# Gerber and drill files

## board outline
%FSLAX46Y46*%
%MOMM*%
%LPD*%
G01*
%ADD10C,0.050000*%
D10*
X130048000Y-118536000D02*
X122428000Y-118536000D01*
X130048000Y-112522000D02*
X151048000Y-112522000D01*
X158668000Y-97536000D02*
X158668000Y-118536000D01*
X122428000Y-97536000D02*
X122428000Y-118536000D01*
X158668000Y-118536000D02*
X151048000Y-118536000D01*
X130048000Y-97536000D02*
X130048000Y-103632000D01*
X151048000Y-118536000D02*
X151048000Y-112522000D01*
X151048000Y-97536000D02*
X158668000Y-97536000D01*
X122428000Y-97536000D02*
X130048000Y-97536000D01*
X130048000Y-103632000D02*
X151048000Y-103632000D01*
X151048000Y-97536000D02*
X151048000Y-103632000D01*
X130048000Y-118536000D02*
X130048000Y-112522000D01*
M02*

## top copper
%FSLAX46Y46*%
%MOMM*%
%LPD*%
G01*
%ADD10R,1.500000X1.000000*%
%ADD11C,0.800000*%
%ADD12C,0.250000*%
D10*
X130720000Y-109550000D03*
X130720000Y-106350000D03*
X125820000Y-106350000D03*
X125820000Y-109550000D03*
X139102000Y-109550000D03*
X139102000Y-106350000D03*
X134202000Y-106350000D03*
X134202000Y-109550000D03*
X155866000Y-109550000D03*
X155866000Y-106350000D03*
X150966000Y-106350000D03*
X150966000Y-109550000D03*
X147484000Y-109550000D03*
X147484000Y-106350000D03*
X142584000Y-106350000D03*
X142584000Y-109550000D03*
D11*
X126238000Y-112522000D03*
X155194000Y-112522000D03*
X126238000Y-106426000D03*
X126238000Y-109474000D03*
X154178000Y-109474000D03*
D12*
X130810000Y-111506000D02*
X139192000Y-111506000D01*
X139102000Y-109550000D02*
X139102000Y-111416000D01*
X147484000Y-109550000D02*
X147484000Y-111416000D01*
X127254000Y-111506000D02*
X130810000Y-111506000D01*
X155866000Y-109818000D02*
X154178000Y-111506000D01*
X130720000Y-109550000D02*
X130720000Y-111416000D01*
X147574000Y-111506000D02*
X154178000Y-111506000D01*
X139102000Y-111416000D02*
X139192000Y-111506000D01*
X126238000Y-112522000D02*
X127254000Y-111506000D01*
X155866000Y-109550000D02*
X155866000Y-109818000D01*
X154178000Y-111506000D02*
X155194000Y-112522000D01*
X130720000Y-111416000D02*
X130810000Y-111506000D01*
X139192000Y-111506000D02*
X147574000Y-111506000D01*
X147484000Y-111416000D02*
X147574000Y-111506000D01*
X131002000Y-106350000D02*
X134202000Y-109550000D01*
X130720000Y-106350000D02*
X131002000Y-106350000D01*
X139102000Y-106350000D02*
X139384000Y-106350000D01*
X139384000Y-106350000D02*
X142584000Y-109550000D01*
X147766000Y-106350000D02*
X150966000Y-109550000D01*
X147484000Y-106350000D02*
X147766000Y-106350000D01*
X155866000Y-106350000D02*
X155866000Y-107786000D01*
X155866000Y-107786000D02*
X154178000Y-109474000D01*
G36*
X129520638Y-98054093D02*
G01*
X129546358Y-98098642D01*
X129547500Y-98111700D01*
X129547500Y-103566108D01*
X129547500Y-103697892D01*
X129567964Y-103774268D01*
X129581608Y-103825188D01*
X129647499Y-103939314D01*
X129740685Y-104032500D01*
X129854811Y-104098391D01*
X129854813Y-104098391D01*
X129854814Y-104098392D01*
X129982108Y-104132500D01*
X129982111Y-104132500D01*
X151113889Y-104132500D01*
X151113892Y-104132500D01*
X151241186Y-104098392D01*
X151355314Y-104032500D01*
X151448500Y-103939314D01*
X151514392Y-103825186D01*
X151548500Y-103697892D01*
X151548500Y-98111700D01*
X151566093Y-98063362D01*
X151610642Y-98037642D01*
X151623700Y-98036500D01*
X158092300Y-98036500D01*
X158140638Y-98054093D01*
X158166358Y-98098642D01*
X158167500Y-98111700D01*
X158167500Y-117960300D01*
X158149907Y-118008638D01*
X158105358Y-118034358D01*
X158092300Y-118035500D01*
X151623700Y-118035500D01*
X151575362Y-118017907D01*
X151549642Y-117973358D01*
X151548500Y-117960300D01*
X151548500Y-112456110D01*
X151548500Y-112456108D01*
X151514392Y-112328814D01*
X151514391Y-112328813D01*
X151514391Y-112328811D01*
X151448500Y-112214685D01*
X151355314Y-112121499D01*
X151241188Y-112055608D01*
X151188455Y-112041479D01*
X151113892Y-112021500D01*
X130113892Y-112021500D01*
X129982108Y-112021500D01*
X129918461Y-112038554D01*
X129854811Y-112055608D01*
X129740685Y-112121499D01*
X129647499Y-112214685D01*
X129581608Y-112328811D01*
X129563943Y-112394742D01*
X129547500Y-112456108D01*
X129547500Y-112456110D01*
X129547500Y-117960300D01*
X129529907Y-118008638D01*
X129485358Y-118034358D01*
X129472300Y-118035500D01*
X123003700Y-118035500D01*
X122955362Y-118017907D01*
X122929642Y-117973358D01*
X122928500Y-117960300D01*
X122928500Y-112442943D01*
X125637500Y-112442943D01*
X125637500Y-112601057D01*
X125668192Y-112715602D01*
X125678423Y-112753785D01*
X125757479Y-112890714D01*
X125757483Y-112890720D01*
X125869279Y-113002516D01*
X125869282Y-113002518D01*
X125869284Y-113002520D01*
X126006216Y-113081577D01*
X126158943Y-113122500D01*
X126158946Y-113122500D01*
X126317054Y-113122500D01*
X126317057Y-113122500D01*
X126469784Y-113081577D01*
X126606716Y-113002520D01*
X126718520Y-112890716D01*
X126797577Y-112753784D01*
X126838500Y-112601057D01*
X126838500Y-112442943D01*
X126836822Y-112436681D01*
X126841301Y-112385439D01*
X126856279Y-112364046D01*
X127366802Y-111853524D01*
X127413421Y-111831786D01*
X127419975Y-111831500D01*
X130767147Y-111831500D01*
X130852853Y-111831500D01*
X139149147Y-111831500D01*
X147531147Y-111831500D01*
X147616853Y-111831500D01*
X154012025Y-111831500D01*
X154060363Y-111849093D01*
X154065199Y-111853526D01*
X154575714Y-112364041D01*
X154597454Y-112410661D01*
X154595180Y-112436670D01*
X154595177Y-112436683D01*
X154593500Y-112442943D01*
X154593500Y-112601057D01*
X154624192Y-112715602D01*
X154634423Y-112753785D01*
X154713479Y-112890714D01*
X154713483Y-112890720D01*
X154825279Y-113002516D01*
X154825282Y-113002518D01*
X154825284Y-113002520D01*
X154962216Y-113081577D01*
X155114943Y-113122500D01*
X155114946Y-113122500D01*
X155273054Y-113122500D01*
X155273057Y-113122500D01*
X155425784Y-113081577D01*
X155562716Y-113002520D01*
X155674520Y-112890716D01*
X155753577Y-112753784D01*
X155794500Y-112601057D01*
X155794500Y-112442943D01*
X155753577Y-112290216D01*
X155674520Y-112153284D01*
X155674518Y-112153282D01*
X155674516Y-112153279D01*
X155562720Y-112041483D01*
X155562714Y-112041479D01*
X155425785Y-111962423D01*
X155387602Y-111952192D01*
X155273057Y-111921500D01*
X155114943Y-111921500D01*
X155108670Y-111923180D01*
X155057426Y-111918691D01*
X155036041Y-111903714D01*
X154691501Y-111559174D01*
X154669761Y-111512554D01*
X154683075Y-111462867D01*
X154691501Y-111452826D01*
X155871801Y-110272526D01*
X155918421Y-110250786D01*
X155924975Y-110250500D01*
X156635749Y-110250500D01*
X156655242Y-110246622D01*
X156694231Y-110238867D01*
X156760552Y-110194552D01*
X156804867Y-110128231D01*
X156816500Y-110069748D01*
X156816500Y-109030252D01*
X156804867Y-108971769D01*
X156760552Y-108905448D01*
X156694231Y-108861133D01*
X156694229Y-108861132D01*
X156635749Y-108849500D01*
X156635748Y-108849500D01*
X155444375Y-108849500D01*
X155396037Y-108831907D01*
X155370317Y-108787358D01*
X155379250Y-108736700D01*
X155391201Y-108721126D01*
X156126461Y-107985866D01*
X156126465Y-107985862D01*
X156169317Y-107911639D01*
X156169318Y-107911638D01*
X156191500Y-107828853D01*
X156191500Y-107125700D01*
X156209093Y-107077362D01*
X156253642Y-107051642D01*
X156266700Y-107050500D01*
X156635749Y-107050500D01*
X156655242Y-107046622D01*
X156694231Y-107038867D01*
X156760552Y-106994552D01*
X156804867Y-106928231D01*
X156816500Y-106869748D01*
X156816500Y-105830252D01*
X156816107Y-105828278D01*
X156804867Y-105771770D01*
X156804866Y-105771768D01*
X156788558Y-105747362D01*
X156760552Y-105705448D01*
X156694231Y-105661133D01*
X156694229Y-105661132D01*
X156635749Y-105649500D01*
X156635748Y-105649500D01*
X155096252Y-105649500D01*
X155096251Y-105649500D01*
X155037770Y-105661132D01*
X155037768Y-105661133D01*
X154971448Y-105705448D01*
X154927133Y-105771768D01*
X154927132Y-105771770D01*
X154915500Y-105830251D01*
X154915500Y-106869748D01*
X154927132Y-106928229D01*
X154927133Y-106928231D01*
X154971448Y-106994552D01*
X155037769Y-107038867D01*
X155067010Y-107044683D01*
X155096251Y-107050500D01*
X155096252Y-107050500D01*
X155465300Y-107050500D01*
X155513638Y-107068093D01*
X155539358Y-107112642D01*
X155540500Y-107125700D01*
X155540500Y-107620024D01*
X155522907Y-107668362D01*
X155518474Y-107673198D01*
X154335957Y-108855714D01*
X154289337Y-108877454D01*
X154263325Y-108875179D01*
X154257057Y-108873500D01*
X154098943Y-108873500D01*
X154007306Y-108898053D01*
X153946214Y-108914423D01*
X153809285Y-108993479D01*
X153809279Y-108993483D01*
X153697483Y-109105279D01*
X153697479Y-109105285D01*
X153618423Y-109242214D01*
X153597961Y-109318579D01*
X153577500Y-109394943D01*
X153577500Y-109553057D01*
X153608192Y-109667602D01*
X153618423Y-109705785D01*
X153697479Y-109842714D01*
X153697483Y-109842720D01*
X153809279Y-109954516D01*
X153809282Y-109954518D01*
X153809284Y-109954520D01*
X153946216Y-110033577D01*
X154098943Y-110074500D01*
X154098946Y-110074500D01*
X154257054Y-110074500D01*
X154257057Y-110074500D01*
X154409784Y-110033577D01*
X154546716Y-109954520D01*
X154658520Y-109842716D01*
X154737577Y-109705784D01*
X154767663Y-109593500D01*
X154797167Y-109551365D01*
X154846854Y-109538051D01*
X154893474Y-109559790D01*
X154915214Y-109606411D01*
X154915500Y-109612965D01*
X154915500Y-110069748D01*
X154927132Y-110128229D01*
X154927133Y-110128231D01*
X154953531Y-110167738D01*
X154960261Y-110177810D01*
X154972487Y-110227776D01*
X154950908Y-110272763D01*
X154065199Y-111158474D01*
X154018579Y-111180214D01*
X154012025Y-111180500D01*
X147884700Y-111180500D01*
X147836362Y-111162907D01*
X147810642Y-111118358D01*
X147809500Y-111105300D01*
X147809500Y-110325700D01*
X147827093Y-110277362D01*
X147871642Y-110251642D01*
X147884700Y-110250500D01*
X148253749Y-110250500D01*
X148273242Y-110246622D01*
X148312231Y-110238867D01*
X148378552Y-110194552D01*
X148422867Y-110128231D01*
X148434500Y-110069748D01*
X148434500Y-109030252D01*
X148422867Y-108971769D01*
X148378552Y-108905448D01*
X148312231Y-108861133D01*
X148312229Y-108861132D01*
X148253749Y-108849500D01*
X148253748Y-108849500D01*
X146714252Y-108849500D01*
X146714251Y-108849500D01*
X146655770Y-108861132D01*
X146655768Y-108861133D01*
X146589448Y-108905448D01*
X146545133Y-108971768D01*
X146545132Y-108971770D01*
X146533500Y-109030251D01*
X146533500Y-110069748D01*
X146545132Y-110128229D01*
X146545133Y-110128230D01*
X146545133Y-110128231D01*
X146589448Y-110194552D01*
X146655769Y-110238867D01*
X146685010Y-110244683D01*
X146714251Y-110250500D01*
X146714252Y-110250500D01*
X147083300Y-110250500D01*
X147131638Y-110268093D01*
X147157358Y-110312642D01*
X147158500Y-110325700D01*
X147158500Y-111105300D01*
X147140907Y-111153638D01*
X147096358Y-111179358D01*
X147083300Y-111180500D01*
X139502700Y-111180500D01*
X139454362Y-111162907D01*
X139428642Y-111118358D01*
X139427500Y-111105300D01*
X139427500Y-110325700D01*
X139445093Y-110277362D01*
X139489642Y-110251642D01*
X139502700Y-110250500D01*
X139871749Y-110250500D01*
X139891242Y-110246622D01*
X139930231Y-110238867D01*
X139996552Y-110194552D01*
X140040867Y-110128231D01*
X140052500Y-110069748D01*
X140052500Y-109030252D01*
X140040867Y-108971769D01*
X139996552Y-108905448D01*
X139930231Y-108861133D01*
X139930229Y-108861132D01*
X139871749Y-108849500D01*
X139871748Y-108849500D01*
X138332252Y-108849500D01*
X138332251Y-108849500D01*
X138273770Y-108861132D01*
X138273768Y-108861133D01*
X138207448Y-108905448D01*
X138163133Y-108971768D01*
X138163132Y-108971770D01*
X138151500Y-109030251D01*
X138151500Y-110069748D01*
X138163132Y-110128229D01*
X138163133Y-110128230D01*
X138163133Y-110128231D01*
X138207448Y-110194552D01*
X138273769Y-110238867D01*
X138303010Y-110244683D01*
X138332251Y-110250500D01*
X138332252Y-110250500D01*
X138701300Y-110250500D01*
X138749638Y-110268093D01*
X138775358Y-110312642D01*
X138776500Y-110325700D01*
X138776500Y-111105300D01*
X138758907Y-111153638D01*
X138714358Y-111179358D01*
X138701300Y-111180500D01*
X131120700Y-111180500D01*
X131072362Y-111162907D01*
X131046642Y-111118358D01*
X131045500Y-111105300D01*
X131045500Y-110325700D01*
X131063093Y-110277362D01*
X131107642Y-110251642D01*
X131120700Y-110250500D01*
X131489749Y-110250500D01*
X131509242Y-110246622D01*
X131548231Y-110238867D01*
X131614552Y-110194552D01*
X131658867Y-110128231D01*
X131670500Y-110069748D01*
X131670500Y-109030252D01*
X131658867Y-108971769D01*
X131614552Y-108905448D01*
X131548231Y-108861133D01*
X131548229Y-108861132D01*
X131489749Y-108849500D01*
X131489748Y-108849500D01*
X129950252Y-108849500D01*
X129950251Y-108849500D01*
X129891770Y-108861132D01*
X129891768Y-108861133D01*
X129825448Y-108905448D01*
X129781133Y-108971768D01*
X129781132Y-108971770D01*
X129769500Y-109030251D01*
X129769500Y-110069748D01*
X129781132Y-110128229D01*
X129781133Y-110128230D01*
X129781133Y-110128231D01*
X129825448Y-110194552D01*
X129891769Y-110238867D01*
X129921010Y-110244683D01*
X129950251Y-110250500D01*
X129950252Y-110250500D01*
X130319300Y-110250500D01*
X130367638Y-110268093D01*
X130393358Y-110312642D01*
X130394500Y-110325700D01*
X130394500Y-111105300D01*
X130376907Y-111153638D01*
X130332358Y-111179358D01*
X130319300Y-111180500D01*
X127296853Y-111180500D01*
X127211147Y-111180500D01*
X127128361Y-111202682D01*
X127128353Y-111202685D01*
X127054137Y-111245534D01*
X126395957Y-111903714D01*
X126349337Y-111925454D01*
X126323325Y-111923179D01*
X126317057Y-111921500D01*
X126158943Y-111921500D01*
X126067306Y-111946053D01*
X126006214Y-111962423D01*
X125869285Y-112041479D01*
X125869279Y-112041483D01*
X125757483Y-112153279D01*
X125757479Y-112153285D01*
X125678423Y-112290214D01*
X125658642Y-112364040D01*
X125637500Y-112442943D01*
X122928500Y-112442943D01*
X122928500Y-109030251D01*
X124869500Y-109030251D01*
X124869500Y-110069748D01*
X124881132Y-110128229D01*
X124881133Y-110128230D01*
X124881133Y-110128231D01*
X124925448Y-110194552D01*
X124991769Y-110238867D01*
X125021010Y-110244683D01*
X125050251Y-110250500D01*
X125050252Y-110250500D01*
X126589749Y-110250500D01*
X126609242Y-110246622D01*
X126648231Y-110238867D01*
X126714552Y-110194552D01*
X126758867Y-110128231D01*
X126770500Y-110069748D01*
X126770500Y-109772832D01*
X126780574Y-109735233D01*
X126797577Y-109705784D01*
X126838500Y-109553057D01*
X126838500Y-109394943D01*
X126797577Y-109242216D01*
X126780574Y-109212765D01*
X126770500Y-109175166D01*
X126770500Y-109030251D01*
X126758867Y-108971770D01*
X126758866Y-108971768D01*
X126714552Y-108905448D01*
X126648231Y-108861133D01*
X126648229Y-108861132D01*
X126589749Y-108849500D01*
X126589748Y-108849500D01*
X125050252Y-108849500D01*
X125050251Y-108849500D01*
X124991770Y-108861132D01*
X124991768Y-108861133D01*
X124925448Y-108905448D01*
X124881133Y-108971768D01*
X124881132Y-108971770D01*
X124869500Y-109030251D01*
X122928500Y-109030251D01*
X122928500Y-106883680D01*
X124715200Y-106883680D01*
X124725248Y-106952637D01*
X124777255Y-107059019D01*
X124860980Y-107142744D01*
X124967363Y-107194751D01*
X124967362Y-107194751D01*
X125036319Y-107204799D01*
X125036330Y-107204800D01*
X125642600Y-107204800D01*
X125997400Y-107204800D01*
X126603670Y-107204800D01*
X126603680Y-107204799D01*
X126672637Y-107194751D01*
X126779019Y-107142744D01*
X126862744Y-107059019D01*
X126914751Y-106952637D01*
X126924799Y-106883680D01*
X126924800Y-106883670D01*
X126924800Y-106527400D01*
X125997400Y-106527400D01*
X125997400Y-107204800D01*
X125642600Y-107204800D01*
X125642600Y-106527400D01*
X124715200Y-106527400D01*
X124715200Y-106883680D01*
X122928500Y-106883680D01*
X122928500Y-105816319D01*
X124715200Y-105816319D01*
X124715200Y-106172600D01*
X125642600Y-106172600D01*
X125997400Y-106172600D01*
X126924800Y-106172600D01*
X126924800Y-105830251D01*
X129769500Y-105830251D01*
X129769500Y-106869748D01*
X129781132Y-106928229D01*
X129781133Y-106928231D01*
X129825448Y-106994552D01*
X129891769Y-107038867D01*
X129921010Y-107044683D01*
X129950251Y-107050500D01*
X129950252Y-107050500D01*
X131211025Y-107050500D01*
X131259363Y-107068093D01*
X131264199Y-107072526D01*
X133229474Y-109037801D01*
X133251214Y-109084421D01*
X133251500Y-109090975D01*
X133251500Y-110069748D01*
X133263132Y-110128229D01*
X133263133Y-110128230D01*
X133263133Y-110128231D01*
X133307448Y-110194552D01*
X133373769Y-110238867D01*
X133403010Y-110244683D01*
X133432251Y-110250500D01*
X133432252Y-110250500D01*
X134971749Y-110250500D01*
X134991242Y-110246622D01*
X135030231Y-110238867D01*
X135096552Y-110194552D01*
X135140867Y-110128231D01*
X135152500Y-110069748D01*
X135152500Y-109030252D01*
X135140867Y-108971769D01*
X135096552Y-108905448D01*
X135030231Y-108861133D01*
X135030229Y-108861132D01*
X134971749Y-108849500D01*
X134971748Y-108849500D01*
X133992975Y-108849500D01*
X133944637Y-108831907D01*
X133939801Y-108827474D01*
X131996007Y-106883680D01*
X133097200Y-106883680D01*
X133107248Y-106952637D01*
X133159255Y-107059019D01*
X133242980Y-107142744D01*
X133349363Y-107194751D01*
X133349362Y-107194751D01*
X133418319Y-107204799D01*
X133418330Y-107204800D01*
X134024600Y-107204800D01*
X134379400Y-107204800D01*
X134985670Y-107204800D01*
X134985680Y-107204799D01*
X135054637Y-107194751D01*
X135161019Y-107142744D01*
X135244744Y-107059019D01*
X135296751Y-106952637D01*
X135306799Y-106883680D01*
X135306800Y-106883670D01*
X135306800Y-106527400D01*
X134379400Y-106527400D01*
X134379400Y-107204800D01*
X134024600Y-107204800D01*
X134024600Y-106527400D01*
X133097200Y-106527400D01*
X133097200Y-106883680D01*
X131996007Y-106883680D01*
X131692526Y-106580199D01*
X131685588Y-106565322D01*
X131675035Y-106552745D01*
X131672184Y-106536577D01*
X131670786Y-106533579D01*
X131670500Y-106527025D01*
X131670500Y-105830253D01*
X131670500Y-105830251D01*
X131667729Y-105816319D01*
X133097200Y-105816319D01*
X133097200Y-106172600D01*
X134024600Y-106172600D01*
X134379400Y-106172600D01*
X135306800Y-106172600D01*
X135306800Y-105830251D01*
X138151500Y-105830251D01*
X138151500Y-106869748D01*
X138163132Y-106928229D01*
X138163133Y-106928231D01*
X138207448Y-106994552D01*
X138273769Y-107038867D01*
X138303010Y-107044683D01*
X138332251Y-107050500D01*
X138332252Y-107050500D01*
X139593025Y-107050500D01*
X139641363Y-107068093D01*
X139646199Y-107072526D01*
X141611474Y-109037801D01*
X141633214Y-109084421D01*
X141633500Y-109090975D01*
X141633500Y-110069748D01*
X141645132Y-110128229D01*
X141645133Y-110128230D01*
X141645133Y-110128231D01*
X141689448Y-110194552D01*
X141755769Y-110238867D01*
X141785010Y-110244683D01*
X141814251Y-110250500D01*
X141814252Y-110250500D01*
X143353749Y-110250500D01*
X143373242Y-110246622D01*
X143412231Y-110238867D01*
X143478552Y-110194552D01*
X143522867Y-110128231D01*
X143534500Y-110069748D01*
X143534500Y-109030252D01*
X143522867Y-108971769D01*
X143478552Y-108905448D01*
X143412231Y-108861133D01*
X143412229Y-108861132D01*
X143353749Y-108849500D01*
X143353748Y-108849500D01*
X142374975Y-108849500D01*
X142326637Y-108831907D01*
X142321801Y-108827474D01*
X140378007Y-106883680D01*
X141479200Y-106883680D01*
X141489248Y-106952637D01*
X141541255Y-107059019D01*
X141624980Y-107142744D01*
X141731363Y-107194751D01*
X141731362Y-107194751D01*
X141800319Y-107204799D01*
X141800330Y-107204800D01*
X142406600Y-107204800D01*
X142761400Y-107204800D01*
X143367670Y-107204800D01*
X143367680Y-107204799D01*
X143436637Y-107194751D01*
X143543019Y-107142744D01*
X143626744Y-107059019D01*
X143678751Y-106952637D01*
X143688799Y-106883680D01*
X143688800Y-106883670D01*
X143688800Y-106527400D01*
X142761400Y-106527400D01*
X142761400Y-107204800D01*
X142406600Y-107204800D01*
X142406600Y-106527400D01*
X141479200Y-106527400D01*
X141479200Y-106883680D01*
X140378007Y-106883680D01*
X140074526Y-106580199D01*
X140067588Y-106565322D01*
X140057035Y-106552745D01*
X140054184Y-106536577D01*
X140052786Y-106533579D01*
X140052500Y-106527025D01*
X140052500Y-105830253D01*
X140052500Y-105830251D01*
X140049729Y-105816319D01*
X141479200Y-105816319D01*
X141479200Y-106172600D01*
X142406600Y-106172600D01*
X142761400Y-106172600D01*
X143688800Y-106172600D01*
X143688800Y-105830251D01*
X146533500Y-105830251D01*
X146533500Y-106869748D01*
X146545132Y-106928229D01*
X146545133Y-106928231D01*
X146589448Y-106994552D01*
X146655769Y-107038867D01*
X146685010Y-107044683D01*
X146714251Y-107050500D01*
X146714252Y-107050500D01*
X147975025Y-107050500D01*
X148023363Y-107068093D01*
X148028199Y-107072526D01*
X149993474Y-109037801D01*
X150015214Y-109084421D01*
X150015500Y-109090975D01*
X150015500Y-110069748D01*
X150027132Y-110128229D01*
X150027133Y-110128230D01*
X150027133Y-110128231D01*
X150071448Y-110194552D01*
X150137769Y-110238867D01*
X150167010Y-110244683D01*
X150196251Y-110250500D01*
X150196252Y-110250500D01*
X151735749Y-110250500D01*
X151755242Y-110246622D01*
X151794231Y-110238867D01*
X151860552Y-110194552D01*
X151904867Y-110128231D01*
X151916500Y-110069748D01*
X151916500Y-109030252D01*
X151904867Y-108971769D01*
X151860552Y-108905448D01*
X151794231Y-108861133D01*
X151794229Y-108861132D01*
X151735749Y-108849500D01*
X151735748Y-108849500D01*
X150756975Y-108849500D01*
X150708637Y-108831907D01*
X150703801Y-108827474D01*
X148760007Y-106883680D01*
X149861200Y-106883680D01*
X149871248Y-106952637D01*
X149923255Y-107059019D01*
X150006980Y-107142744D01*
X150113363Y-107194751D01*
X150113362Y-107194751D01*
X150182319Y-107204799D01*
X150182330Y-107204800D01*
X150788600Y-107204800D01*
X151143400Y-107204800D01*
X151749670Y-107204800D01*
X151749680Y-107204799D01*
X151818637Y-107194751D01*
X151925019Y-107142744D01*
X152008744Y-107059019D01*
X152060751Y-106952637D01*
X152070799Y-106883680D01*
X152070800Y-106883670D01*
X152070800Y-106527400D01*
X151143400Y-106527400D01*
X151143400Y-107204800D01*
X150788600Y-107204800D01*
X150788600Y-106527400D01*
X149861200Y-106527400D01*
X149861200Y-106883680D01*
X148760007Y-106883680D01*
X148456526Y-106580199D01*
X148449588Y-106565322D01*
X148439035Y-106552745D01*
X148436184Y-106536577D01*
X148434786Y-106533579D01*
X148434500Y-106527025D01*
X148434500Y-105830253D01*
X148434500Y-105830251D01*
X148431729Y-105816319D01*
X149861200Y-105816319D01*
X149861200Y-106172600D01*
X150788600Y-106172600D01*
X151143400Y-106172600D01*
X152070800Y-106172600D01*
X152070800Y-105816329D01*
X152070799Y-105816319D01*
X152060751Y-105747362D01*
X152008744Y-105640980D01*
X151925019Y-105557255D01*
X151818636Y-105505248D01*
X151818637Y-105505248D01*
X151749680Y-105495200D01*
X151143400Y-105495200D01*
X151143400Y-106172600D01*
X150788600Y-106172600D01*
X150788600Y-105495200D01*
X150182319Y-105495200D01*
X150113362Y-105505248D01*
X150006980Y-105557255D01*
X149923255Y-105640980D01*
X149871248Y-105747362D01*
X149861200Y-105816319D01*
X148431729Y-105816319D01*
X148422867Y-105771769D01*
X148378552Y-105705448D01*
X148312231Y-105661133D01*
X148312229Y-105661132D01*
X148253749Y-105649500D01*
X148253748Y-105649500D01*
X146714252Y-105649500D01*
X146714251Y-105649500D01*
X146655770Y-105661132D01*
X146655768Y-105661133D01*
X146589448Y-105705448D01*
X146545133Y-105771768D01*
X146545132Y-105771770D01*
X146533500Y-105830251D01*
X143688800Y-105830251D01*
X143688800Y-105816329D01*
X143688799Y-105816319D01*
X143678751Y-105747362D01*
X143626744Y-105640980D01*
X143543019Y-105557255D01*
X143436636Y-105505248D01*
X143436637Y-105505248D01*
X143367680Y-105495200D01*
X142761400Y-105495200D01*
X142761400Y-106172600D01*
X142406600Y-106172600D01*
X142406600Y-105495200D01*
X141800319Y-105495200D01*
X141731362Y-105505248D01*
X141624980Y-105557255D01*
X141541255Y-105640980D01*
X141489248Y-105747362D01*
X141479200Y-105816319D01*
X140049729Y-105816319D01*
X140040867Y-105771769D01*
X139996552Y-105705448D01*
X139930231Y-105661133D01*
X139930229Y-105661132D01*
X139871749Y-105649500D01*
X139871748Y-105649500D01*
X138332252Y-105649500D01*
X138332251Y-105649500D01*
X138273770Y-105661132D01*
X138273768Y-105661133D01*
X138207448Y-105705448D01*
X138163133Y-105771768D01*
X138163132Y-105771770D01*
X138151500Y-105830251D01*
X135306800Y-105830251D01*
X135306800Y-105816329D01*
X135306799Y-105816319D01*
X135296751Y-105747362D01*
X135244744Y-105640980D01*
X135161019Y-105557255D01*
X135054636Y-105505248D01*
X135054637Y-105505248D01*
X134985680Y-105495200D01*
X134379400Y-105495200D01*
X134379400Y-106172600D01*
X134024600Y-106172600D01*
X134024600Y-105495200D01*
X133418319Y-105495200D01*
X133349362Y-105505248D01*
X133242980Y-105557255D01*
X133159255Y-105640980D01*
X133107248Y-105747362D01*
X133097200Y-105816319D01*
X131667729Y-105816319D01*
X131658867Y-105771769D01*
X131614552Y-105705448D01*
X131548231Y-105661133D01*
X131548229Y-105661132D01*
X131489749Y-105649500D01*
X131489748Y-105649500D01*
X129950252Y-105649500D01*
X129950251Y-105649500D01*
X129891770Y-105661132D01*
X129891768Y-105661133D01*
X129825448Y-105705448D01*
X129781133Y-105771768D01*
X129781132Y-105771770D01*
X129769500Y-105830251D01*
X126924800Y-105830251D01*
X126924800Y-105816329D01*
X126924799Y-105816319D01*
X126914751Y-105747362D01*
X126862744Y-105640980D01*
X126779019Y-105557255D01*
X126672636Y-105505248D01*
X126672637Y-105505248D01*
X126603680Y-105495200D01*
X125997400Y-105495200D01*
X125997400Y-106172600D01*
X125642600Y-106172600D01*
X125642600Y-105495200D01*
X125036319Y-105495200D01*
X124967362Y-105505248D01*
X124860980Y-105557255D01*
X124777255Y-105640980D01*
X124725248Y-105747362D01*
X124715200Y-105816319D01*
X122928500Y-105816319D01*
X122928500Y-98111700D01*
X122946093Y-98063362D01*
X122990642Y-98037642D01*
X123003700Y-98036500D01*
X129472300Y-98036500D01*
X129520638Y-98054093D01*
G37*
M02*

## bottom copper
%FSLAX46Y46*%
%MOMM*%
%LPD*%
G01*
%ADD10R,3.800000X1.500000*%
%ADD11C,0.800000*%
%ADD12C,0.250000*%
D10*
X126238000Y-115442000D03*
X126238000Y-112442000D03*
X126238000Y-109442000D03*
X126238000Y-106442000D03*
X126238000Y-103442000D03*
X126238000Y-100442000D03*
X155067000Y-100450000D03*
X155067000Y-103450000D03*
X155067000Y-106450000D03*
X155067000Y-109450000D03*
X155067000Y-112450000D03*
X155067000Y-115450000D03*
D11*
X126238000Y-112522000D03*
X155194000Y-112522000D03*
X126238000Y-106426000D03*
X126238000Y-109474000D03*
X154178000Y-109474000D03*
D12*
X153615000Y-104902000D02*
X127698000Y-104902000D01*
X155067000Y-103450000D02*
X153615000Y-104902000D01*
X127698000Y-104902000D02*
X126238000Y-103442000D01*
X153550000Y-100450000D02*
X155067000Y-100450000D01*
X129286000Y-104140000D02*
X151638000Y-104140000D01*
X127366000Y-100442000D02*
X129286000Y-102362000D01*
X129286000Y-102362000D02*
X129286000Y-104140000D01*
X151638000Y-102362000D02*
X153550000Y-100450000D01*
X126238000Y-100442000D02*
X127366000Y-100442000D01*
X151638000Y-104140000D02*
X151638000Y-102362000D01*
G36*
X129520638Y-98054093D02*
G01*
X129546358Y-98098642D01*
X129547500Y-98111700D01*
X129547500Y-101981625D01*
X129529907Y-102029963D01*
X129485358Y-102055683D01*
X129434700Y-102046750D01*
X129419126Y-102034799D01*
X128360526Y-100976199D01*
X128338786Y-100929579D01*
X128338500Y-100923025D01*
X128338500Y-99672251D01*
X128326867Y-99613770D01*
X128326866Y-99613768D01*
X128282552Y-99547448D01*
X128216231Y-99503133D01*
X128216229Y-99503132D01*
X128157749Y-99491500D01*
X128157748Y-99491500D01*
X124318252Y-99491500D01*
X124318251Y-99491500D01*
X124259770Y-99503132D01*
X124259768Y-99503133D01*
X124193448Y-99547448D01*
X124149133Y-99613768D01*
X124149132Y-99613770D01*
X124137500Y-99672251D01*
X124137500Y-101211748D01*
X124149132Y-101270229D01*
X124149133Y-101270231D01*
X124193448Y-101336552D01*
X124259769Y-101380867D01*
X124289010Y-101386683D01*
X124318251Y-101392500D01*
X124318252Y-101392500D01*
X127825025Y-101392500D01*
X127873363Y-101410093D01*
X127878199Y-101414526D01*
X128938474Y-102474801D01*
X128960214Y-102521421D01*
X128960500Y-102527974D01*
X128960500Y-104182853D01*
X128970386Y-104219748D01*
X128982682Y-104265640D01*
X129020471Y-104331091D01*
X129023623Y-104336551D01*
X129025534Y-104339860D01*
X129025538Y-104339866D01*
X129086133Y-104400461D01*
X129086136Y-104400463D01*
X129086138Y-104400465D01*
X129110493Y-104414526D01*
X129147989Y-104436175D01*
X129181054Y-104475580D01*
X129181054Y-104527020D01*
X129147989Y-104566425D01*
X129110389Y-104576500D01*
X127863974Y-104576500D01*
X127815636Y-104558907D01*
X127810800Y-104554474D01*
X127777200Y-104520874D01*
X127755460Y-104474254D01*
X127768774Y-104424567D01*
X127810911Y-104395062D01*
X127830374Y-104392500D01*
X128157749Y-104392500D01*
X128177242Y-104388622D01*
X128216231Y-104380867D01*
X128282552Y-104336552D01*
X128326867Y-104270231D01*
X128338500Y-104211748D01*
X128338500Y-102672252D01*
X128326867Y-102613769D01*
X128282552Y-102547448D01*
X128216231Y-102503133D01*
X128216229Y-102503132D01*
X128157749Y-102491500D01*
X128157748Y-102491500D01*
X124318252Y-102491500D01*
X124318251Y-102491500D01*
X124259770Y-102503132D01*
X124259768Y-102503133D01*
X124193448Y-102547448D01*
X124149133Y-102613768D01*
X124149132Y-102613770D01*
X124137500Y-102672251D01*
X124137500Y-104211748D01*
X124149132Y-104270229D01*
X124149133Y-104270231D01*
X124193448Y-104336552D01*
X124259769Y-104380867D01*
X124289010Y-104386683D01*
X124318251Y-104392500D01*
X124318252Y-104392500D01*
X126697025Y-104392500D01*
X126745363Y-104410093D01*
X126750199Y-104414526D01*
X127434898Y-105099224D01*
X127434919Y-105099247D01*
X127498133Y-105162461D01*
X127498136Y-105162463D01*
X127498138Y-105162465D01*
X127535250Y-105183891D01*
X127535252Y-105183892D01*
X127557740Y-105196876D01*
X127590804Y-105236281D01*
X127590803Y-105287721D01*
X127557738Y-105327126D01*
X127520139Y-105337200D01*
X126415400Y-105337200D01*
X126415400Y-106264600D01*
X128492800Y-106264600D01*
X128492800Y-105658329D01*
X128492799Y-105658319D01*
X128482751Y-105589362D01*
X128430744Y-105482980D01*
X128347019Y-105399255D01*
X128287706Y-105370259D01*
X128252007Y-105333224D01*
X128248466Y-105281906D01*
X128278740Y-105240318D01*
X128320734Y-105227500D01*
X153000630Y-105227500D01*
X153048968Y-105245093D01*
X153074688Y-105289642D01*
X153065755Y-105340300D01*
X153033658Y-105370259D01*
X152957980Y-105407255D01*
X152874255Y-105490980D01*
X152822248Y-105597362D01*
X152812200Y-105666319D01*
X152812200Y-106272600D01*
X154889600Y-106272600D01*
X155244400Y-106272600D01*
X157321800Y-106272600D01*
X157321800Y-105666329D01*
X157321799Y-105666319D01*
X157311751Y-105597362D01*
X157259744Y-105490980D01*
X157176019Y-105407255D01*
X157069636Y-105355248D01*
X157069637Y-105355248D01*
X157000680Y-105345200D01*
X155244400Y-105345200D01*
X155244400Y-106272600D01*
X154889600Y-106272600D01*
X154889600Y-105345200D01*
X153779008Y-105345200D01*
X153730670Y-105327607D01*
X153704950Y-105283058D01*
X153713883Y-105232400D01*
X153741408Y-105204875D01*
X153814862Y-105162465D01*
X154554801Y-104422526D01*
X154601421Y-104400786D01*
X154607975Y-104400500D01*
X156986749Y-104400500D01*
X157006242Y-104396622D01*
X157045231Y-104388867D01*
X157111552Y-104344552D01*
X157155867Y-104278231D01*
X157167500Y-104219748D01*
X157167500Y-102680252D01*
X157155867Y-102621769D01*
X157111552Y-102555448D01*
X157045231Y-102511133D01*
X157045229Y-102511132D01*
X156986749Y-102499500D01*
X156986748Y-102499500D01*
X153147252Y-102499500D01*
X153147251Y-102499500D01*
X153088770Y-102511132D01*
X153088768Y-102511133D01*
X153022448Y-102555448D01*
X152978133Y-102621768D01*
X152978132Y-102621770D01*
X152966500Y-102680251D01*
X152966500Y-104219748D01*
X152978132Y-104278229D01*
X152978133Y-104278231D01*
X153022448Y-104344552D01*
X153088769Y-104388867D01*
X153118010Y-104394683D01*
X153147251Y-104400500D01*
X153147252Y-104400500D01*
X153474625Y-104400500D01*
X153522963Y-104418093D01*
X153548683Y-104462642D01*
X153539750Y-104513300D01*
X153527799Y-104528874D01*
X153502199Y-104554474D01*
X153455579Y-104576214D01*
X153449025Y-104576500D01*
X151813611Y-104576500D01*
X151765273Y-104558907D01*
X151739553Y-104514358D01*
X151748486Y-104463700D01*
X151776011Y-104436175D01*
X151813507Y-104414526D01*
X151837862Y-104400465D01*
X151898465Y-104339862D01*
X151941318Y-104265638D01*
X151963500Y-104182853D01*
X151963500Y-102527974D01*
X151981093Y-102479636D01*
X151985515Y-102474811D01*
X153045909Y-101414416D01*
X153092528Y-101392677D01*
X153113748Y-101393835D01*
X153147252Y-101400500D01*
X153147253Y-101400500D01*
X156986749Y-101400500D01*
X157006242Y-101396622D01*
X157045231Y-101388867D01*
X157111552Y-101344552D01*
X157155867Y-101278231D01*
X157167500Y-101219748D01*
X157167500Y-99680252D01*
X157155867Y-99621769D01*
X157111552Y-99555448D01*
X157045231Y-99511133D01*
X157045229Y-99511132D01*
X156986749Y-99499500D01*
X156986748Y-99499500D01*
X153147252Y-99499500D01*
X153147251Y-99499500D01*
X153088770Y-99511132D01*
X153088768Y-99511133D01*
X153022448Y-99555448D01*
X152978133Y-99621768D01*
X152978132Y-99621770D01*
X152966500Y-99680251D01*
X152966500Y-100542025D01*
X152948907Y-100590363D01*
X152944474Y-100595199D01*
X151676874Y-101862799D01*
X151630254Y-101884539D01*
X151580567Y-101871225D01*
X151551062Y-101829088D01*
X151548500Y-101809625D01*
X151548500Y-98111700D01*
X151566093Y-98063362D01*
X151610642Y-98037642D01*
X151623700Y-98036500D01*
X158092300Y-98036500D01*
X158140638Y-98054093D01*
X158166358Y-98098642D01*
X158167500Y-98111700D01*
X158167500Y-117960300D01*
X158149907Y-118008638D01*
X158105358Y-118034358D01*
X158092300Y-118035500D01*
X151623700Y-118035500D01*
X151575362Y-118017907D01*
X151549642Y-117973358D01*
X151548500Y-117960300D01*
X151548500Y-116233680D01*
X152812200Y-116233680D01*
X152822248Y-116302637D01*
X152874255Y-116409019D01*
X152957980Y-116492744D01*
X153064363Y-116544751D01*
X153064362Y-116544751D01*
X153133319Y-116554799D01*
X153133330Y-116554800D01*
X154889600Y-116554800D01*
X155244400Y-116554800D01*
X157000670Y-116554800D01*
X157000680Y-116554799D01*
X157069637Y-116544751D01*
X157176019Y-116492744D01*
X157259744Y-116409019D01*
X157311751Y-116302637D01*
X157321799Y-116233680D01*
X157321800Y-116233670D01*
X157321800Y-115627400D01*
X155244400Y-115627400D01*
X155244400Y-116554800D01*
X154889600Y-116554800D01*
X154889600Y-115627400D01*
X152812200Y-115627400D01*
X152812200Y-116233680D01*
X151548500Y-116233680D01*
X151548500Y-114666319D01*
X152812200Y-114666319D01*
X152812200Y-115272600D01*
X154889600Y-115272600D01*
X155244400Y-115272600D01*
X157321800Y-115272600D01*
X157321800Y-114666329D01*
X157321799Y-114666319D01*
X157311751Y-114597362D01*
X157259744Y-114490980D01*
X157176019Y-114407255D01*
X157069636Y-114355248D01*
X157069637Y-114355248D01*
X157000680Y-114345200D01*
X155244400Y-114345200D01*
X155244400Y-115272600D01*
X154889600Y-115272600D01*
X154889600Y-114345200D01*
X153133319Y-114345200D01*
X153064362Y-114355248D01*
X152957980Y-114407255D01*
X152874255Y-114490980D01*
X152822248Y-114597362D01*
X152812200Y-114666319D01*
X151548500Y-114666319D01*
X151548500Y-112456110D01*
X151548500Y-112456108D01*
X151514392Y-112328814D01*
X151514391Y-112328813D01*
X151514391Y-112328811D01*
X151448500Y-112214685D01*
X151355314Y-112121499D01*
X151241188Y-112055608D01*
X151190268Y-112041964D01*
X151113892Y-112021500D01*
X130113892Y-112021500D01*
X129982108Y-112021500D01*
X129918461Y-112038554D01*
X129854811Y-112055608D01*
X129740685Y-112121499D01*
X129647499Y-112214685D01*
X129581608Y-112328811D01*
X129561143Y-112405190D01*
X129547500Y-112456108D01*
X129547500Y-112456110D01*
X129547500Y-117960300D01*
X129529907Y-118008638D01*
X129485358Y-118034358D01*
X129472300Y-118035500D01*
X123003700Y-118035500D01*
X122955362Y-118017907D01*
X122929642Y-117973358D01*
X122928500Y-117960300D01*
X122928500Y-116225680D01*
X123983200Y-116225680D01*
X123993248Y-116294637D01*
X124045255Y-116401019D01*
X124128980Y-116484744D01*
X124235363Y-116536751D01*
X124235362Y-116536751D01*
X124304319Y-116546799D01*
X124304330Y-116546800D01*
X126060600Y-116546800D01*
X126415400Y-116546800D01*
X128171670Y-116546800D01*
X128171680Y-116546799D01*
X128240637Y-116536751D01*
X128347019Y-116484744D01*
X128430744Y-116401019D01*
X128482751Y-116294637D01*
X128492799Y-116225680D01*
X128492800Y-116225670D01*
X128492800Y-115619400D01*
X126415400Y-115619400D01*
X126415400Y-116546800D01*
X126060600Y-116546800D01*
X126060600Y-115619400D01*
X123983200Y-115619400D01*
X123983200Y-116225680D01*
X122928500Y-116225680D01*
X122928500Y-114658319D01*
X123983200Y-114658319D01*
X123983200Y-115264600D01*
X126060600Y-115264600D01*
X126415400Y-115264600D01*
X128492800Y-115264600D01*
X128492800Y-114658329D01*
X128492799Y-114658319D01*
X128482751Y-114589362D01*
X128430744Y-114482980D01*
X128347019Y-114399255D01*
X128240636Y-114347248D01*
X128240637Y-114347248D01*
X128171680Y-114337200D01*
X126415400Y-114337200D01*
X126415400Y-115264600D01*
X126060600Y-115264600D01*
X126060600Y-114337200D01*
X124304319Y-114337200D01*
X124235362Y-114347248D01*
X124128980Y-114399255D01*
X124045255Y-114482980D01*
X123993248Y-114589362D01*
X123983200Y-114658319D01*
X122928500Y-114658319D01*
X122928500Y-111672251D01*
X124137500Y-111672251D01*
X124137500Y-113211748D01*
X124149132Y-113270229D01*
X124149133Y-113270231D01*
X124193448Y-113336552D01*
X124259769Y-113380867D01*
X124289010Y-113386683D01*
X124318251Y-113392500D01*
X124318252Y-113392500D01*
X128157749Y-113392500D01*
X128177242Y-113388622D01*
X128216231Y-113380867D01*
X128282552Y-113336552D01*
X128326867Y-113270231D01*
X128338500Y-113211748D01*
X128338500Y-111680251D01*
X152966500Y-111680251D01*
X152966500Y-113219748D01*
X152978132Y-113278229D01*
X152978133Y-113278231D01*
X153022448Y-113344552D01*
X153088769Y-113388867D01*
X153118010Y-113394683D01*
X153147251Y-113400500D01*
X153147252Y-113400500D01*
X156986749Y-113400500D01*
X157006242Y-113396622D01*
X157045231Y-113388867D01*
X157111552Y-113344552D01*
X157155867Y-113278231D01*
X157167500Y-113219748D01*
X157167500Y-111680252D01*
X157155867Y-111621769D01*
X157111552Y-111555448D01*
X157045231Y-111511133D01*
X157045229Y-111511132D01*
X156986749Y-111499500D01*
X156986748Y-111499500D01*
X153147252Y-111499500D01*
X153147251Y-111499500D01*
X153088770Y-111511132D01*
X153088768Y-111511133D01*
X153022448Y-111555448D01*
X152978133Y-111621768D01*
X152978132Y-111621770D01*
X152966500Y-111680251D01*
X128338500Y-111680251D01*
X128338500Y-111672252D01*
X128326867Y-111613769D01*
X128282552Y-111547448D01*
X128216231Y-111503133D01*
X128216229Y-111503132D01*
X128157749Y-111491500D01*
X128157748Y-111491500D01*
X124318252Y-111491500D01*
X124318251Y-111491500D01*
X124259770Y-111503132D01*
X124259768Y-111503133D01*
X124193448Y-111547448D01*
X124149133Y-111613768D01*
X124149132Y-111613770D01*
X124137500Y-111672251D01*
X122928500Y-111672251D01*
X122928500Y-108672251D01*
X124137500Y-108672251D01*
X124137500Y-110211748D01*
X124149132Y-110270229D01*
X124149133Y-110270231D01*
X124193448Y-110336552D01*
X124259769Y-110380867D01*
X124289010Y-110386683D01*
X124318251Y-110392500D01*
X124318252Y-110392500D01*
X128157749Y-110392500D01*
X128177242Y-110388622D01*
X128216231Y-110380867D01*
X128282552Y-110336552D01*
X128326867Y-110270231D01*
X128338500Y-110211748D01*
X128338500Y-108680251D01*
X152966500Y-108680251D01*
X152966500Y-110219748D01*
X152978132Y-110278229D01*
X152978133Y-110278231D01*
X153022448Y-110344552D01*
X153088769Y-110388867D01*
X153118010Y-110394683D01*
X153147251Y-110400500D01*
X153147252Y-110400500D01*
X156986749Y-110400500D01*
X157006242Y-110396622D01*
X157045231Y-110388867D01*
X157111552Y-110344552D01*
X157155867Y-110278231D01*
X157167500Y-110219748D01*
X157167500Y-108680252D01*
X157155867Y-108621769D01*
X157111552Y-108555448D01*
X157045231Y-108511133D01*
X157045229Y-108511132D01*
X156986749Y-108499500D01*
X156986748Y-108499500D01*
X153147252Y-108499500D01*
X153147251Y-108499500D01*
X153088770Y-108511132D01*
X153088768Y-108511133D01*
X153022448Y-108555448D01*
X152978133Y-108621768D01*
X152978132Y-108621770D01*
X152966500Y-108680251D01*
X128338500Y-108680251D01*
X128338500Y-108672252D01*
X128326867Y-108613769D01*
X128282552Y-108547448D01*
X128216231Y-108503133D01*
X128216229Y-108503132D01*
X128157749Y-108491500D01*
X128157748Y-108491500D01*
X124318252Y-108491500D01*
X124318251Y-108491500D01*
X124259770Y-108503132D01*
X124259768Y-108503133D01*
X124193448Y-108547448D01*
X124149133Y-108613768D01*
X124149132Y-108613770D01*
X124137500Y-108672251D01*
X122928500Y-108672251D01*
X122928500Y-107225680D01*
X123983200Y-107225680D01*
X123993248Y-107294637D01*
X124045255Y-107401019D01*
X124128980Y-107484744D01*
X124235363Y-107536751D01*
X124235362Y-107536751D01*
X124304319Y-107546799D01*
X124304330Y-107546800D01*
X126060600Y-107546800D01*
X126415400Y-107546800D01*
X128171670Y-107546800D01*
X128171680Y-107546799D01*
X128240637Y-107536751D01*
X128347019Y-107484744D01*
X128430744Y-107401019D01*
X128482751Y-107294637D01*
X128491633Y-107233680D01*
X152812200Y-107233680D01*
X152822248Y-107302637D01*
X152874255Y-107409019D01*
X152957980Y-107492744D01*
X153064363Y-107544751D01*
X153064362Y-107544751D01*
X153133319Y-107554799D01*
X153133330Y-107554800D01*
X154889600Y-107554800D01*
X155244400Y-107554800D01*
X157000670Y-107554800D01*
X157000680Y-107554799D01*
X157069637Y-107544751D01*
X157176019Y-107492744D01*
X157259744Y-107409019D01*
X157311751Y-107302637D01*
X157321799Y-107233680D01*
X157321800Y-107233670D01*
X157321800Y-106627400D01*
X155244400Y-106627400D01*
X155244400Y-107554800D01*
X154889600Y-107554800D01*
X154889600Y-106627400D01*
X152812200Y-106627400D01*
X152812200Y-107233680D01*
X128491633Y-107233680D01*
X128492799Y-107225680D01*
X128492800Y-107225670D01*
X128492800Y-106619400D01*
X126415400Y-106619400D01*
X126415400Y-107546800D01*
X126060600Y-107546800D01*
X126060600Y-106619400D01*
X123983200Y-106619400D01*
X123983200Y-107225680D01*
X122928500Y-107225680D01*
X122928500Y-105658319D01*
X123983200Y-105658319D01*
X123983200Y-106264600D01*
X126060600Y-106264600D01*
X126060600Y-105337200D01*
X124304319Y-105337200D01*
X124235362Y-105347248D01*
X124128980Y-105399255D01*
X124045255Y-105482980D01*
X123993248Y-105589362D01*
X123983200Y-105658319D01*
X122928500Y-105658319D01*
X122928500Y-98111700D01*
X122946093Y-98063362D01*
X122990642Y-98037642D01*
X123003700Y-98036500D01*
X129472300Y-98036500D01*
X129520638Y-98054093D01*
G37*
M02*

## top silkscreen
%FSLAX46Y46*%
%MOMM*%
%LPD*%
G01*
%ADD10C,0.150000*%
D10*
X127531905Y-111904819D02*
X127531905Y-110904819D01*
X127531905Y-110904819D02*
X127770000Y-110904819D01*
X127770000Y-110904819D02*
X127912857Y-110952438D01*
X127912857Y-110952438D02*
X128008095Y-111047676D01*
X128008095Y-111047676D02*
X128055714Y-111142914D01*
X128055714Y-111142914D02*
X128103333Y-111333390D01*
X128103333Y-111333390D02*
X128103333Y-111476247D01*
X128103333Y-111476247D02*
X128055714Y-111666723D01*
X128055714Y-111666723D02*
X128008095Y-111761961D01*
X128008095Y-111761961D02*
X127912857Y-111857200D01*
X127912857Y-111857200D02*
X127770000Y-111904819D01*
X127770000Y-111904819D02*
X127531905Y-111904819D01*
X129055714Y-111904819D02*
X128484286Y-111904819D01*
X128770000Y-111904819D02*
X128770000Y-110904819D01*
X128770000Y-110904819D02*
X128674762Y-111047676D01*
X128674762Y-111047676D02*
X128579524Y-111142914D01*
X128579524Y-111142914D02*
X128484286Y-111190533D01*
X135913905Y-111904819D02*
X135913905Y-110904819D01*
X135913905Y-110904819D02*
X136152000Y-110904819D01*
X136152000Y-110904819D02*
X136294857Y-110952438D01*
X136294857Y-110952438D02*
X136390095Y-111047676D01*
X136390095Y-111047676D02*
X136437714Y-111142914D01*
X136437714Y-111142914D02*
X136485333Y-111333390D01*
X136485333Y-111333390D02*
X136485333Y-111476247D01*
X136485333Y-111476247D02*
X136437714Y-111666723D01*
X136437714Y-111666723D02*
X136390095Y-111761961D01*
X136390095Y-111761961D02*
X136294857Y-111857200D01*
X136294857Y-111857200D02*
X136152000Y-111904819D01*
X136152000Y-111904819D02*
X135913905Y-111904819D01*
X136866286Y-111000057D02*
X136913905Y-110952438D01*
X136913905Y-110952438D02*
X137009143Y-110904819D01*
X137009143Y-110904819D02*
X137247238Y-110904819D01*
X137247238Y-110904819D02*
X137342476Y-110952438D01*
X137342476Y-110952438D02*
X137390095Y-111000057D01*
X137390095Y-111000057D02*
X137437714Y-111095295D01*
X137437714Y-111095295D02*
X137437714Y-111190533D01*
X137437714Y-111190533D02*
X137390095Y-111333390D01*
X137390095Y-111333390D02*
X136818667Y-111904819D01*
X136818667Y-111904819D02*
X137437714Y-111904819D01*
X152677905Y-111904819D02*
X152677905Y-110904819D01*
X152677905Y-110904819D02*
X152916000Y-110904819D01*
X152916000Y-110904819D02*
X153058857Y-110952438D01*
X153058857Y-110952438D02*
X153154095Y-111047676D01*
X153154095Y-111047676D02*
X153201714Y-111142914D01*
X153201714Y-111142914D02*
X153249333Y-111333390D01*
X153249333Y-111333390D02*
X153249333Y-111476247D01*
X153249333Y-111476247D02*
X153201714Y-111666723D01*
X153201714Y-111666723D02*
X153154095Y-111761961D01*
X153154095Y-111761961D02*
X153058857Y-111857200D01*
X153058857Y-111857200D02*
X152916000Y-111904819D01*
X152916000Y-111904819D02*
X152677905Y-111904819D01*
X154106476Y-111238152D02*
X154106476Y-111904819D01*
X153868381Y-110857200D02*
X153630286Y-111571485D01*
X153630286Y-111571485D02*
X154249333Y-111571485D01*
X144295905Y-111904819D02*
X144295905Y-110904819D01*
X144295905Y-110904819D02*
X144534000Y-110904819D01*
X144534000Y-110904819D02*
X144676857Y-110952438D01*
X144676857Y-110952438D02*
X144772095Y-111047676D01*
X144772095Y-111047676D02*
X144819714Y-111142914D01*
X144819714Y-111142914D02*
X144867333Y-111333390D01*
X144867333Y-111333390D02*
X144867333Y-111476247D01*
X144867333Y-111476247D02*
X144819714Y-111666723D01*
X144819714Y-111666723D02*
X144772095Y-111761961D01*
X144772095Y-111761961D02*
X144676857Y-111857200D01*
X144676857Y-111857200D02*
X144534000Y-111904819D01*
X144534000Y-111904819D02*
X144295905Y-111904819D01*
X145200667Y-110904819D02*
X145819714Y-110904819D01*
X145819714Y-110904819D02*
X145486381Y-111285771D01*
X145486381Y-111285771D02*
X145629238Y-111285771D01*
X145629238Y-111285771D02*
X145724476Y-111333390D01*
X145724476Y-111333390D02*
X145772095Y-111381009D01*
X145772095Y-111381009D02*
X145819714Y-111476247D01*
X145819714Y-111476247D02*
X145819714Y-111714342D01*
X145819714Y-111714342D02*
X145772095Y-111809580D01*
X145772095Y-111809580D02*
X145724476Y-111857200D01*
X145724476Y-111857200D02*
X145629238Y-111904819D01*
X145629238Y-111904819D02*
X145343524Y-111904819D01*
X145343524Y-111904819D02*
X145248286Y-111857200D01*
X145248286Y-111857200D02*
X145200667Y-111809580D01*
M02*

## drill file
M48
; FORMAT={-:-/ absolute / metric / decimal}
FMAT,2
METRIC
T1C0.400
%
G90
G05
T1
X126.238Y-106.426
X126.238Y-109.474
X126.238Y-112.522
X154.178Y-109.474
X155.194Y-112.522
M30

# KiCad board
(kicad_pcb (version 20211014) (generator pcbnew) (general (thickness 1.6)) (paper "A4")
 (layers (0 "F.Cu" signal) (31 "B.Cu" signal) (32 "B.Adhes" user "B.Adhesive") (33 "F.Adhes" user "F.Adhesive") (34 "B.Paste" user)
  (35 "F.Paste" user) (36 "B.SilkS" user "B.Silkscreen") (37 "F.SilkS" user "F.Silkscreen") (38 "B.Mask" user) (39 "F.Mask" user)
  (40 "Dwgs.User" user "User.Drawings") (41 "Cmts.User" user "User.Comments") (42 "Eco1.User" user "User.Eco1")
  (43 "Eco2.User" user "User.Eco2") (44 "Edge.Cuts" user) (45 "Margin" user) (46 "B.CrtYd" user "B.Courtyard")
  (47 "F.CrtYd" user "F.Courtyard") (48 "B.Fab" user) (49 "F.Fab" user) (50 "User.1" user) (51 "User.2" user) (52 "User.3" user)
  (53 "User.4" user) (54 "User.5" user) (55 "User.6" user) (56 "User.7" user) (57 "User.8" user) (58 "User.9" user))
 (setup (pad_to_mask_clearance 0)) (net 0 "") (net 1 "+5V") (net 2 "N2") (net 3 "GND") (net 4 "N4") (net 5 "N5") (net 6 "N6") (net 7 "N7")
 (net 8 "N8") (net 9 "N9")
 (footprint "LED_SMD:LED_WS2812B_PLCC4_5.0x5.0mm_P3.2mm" (layer "F.Cu") (at 128.27 107.95 180)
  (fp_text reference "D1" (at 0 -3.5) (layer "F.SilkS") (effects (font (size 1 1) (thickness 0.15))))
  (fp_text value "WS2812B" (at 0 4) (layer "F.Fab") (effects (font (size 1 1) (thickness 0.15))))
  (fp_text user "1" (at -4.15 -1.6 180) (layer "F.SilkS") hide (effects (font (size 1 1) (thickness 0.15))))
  (pad "1" smd rect (at -2.45 -1.6 180) (size 1.5 1) (layers "F.Cu" "F.Paste" "F.Mask") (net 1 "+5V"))
  (pad "2" smd rect (at -2.45 1.6 180) (size 1.5 1) (layers "F.Cu" "F.Paste" "F.Mask") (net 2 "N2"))
  (pad "3" smd rect (at 2.45 1.6 180) (size 1.5 1) (layers "F.Cu" "F.Paste" "F.Mask") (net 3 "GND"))
  (pad "4" smd rect (at 2.45 -1.6 180) (size 1.5 1) (layers "F.Cu" "F.Paste" "F.Mask") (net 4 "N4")))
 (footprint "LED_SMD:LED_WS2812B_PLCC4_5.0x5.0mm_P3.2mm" (layer "F.Cu") (at 136.652 107.95 180)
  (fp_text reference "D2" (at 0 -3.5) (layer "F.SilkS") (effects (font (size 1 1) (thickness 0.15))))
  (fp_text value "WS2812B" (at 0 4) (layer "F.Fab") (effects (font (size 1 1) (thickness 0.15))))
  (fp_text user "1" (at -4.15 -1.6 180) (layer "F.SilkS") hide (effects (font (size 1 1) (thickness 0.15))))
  (pad "1" smd rect (at -2.45 -1.6 180) (size 1.5 1) (layers "F.Cu" "F.Paste" "F.Mask") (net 1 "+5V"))
  (pad "2" smd rect (at -2.45 1.6 180) (size 1.5 1) (layers "F.Cu" "F.Paste" "F.Mask") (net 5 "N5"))
  (pad "3" smd rect (at 2.45 1.6 180) (size 1.5 1) (layers "F.Cu" "F.Paste" "F.Mask") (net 3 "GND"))
  (pad "4" smd rect (at 2.45 -1.6 180) (size 1.5 1) (layers "F.Cu" "F.Paste" "F.Mask") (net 2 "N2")))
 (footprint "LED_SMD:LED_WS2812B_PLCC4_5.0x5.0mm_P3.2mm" (layer "F.Cu") (at 153.416 107.95 180)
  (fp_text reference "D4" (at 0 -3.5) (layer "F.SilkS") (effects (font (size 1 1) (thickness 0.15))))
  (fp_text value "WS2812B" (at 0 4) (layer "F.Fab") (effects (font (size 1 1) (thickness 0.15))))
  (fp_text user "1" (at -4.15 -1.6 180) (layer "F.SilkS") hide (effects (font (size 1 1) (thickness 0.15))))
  (pad "1" smd rect (at -2.45 -1.6 180) (size 1.5 1) (layers "F.Cu" "F.Paste" "F.Mask") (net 1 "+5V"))
  (pad "2" smd rect (at -2.45 1.6 180) (size 1.5 1) (layers "F.Cu" "F.Paste" "F.Mask") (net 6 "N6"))
  (pad "3" smd rect (at 2.45 1.6 180) (size 1.5 1) (layers "F.Cu" "F.Paste" "F.Mask") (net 3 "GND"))
  (pad "4" smd rect (at 2.45 -1.6 180) (size 1.5 1) (layers "F.Cu" "F.Paste" "F.Mask") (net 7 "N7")))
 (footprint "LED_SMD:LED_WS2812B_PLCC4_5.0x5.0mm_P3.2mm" (layer "F.Cu") (at 145.034 107.95 180)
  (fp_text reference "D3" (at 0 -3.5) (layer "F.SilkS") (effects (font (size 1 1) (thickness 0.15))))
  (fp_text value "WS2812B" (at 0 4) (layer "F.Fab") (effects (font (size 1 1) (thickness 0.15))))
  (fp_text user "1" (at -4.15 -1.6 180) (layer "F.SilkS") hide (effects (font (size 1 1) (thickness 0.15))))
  (pad "1" smd rect (at -2.45 -1.6 180) (size 1.5 1) (layers "F.Cu" "F.Paste" "F.Mask") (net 1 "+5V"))
  (pad "2" smd rect (at -2.45 1.6 180) (size 1.5 1) (layers "F.Cu" "F.Paste" "F.Mask") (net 7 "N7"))
  (pad "3" smd rect (at 2.45 1.6 180) (size 1.5 1) (layers "F.Cu" "F.Paste" "F.Mask") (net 3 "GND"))
  (pad "4" smd rect (at 2.45 -1.6 180) (size 1.5 1) (layers "F.Cu" "F.Paste" "F.Mask") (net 5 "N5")))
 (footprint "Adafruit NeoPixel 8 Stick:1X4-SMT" (layer "B.Cu") (at 126.873 107.442 90)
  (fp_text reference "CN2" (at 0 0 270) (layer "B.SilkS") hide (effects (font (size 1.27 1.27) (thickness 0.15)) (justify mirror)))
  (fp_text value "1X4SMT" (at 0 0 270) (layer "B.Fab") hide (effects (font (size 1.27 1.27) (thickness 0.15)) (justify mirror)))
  (pad "1" smd rect (at -8 -0.635 90) (size 1.5 3.8) (layers "B.Cu" "B.Paste" "B.Mask") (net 3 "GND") (solder_mask_margin 0.1016))
  (pad "2" smd rect (at -5 -0.635 90) (size 1.5 3.8) (layers "B.Cu" "B.Paste" "B.Mask") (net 1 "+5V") (solder_mask_margin 0.1016))
  (pad "3" smd rect (at -2 -0.635 90) (size 1.5 3.8) (layers "B.Cu" "B.Paste" "B.Mask") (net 4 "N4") (solder_mask_margin 0.1016))
  (pad "4" smd rect (at 1 -0.635 90) (size 1.5 3.8) (layers "B.Cu" "B.Paste" "B.Mask") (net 3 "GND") (solder_mask_margin 0.1016))
  (pad "5" smd rect (at 4 -0.635 90) (size 1.5 3.8) (layers "B.Cu" "B.Paste" "B.Mask") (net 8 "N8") (solder_mask_margin 0.1016))
  (pad "6" smd rect (at 7 -0.635 90) (size 1.5 3.8) (layers "B.Cu" "B.Paste" "B.Mask") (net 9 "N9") (solder_mask_margin 0.1016)))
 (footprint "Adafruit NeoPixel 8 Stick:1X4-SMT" (layer "B.Cu") (at 154.432 108.45 -90)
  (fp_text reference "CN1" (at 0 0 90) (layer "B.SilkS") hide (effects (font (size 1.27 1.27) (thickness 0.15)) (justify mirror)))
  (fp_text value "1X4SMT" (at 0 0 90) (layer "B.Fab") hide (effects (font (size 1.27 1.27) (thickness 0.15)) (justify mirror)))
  (pad "1" smd rect (at -8 -0.635 270) (size 1.5 3.8) (layers "B.Cu" "B.Paste" "B.Mask") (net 9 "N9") (solder_mask_margin 0.1016))
  (pad "2" smd rect (at -5 -0.635 270) (size 1.5 3.8) (layers "B.Cu" "B.Paste" "B.Mask") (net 8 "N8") (solder_mask_margin 0.1016))
  (pad "3" smd rect (at -2 -0.635 270) (size 1.5 3.8) (layers "B.Cu" "B.Paste" "B.Mask") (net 3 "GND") (solder_mask_margin 0.1016))
  (pad "4" smd rect (at 1 -0.635 270) (size 1.5 3.8) (layers "B.Cu" "B.Paste" "B.Mask") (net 6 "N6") (solder_mask_margin 0.1016))
  (pad "5" smd rect (at 4 -0.635 270) (size 1.5 3.8) (layers "B.Cu" "B.Paste" "B.Mask") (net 1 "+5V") (solder_mask_margin 0.1016))
  (pad "6" smd rect (at 7 -0.635 270) (size 1.5 3.8) (layers "B.Cu" "B.Paste" "B.Mask") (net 3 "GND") (solder_mask_margin 0.1016)))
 (gr_line (start 130.048 118.536) (end 122.428 118.536) (layer "Edge.Cuts") (width 0.05))
 (gr_line (start 130.048 112.522) (end 151.048 112.522) (layer "Edge.Cuts") (width 0.05))
 (gr_line (start 158.668 97.536) (end 158.668 118.536) (layer "Edge.Cuts") (width 0.05))
 (gr_line (start 122.428 97.536) (end 122.428 118.536) (layer "Edge.Cuts") (width 0.05))
 (gr_line locked (start 158.668 118.536) (end 151.048 118.536) (layer "Edge.Cuts") (width 0.05))
 (gr_line (start 130.048 97.536) (end 130.048 103.632) (layer "Edge.Cuts") (width 0.05))
 (gr_line (start 151.048 118.536) (end 151.048 112.522) (layer "Edge.Cuts") (width 0.05))
 (gr_line (start 151.048 97.536) (end 158.668 97.536) (layer "Edge.Cuts") (width 0.05))
 (gr_line (start 122.428 97.536) (end 130.048 97.536) (layer "Edge.Cuts") (width 0.05))
 (gr_line (start 130.048 103.632) (end 151.048 103.632) (layer "Edge.Cuts") (width 0.05))
 (gr_line (start 151.048 97.536) (end 151.048 103.632) (layer "Edge.Cuts") (width 0.05))
 (gr_line (start 130.048 118.536) (end 130.048 112.522) (layer "Edge.Cuts") (width 0.05))
 (segment (start 130.81 111.506) (end 139.192 111.506) (width 0.25) (layer "F.Cu") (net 1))
 (segment (start 139.102 109.55) (end 139.102 111.416) (width 0.25) (layer "F.Cu") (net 1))
 (segment (start 147.484 109.55) (end 147.484 111.416) (width 0.25) (layer "F.Cu") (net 1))
 (segment (start 127.254 111.506) (end 130.81 111.506) (width 0.25) (layer "F.Cu") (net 1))
 (segment (start 155.866 109.818) (end 154.178 111.506) (width 0.25) (layer "F.Cu") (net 1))
 (segment (start 130.72 109.55) (end 130.72 111.416) (width 0.25) (layer "F.Cu") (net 1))
 (segment (start 147.574 111.506) (end 154.178 111.506) (width 0.25) (layer "F.Cu") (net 1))
 (segment (start 139.102 111.416) (end 139.192 111.506) (width 0.25) (layer "F.Cu") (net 1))
 (segment (start 126.238 112.522) (end 127.254 111.506) (width 0.25) (layer "F.Cu") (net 1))
 (segment (start 155.866 109.55) (end 155.866 109.818) (width 0.25) (layer "F.Cu") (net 1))
 (segment (start 154.178 111.506) (end 155.194 112.522) (width 0.25) (layer "F.Cu") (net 1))
 (segment (start 130.72 111.416) (end 130.81 111.506) (width 0.25) (layer "F.Cu") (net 1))
 (segment (start 139.192 111.506) (end 147.574 111.506) (width 0.25) (layer "F.Cu") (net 1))
 (segment (start 147.484 111.416) (end 147.574 111.506) (width 0.25) (layer "F.Cu") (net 1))
 (via (at 126.238 112.522) (size 0.8) (drill 0.4) (layers "F.Cu" "B.Cu") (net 1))
 (via (at 155.194 112.522) (size 0.8) (drill 0.4) (layers "F.Cu" "B.Cu") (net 1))
 (via (at 126.238 106.426) (size 0.8) (drill 0.4) (layers "F.Cu" "B.Cu") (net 3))
 (segment (start 153.615 104.902) (end 127.698 104.902) (width 0.25) (layer "B.Cu") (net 8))
 (segment (start 155.067 103.45) (end 153.615 104.902) (width 0.25) (layer "B.Cu") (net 8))
 (segment (start 127.698 104.902) (end 126.238 103.442) (width 0.25) (layer "B.Cu") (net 8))
 (via (at 126.238 109.474) (size 0.8) (drill 0.4) (layers "F.Cu" "B.Cu") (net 4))
 (segment (start 131.002 106.35) (end 134.202 109.55) (width 0.25) (layer "F.Cu") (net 2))
 (segment (start 130.72 106.35) (end 131.002 106.35) (width 0.25) (layer "F.Cu") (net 2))
 (segment (start 139.102 106.35) (end 139.384 106.35) (width 0.25) (layer "F.Cu") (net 5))
 (segment (start 139.384 106.35) (end 142.584 109.55) (width 0.25) (layer "F.Cu") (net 5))
 (segment (start 147.766 106.35) (end 150.966 109.55) (width 0.25) (layer "F.Cu") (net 7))
 (segment (start 147.484 106.35) (end 147.766 106.35) (width 0.25) (layer "F.Cu") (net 7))
 (segment (start 155.866 106.35) (end 155.866 107.786) (width 0.25) (layer "F.Cu") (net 6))
 (segment (start 155.866 107.786) (end 154.178 109.474) (width 0.25) (layer "F.Cu") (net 6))
 (via (at 154.178 109.474) (size 0.8) (drill 0.4) (layers "F.Cu" "B.Cu") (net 6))
 (segment (start 153.55 100.45) (end 155.067 100.45) (width 0.25) (layer "B.Cu") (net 9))
 (segment (start 129.286 104.14) (end 151.638 104.14) (width 0.25) (layer "B.Cu") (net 9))
 (segment (start 127.366 100.442) (end 129.286 102.362) (width 0.25) (layer "B.Cu") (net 9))
 (segment (start 129.286 102.362) (end 129.286 104.14) (width 0.25) (layer "B.Cu") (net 9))
 (segment (start 151.638 102.362) (end 153.55 100.45) (width 0.25) (layer "B.Cu") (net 9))
 (segment (start 126.238 100.442) (end 127.366 100.442) (width 0.25) (layer "B.Cu") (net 9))
 (segment (start 151.638 104.14) (end 151.638 102.362) (width 0.25) (layer "B.Cu") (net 9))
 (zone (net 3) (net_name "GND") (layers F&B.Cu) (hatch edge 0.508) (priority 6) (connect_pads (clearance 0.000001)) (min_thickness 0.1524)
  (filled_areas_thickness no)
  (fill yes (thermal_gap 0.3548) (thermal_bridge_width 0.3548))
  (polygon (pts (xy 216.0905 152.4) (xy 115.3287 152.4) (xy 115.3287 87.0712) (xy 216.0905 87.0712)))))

